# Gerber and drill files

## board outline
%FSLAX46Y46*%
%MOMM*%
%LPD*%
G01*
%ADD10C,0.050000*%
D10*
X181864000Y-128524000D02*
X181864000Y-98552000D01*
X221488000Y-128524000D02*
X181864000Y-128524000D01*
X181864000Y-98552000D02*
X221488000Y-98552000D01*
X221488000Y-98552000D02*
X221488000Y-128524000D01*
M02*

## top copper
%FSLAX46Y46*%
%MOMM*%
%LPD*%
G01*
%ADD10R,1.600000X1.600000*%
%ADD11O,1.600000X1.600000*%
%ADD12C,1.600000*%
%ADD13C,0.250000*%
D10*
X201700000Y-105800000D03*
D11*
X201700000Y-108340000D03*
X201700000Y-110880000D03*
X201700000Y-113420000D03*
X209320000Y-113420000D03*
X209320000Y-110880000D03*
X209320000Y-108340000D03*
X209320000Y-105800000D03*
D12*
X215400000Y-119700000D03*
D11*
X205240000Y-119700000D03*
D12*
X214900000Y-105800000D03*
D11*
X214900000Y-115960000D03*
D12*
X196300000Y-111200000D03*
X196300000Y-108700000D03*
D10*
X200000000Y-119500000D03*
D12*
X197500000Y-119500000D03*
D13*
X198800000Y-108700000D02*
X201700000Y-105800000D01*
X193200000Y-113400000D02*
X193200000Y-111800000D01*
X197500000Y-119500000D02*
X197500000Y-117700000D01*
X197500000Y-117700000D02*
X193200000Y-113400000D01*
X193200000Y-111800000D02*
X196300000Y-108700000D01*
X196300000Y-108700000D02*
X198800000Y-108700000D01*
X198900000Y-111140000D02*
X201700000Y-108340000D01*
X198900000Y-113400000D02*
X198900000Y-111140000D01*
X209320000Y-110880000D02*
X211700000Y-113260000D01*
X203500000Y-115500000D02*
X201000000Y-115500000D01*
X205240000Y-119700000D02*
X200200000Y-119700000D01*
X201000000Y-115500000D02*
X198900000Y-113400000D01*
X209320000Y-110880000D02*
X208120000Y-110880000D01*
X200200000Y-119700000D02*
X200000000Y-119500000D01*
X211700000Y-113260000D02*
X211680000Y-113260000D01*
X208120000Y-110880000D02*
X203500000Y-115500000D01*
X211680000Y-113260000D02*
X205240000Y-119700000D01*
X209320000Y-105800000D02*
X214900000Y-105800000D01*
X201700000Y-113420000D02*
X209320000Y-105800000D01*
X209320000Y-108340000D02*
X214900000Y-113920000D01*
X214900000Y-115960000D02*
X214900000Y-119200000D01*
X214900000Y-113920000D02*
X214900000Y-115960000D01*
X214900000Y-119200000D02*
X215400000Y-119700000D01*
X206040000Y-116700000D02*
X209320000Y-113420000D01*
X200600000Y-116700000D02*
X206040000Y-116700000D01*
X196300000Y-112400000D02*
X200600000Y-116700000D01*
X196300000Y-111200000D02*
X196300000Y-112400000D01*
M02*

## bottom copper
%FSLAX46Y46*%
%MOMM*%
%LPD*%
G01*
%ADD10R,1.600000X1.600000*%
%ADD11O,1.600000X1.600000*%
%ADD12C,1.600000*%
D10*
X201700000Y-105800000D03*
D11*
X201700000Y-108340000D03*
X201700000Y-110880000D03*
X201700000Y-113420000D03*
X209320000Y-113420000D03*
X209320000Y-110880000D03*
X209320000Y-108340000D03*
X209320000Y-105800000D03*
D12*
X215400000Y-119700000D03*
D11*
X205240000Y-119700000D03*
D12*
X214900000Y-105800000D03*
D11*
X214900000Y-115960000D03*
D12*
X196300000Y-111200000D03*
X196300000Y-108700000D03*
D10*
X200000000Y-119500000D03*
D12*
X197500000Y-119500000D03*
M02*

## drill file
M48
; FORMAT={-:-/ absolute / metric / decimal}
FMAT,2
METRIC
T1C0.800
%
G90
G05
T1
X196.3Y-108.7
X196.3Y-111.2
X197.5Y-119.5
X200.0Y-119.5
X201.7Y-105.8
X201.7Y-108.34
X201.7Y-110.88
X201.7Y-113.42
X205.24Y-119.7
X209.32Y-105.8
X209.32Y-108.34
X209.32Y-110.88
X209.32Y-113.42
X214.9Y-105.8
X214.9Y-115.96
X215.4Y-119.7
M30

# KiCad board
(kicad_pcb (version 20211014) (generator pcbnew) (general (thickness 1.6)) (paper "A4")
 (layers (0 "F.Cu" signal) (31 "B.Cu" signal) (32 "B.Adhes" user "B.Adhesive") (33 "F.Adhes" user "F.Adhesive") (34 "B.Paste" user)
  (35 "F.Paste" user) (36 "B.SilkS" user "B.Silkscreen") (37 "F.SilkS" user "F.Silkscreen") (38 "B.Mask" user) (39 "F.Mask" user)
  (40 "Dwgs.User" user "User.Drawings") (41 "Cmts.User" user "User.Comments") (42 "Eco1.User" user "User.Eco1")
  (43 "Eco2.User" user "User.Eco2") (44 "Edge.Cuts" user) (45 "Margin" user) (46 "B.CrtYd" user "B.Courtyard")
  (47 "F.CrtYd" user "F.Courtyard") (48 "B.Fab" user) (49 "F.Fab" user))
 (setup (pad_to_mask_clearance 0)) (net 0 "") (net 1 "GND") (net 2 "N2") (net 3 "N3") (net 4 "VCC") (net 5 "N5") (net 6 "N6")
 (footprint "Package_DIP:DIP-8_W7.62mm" (layer "F.Cu") (at 201.7 105.8)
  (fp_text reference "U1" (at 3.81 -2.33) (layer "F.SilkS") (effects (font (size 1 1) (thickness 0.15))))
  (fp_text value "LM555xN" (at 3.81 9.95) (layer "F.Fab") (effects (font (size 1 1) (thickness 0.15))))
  (pad "1" thru_hole rect locked (at 0 0) (size 1.6 1.6) (drill 0.8) (layers *.Cu *.Mask) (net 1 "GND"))
  (pad "2" thru_hole oval locked (at 0 2.54) (size 1.6 1.6) (drill 0.8) (layers *.Cu *.Mask) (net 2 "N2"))
  (pad "3" thru_hole oval locked (at 0 5.08) (size 1.6 1.6) (drill 0.8) (layers *.Cu *.Mask) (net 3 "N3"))
  (pad "4" thru_hole oval locked (at 0 7.62) (size 1.6 1.6) (drill 0.8) (layers *.Cu *.Mask) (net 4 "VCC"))
  (pad "5" thru_hole oval locked (at 7.62 7.62) (size 1.6 1.6) (drill 0.8) (layers *.Cu *.Mask) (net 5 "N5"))
  (pad "6" thru_hole oval locked (at 7.62 5.08) (size 1.6 1.6) (drill 0.8) (layers *.Cu *.Mask) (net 2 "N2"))
  (pad "7" thru_hole oval locked (at 7.62 2.54) (size 1.6 1.6) (drill 0.8) (layers *.Cu *.Mask) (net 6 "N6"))
  (pad "8" thru_hole oval locked (at 7.62 0) (size 1.6 1.6) (drill 0.8) (layers *.Cu *.Mask) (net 4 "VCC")))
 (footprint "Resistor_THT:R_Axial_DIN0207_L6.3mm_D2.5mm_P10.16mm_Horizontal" (layer "F.Cu") (at 215.4 119.7 180)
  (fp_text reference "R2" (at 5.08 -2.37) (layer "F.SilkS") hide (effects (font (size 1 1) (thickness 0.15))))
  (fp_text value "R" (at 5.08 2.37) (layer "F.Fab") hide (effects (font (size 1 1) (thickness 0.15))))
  (pad "1" thru_hole circle locked (at 0 0 180) (size 1.6 1.6) (drill 0.8) (layers *.Cu *.Mask) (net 6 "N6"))
  (pad "2" thru_hole oval locked (at 10.16 0 180) (size 1.6 1.6) (drill 0.8) (layers *.Cu *.Mask) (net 2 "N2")))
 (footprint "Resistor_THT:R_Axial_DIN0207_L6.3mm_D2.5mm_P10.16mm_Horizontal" (layer "F.Cu") (at 214.9 105.8 -90)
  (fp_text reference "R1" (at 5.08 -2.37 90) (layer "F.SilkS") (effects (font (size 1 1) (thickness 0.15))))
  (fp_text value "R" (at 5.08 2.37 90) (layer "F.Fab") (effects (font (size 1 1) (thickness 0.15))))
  (pad "1" thru_hole circle locked (at 0 0 270) (size 1.6 1.6) (drill 0.8) (layers *.Cu *.Mask) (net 4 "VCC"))
  (pad "2" thru_hole oval locked (at 10.16 0 270) (size 1.6 1.6) (drill 0.8) (layers *.Cu *.Mask) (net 6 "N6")))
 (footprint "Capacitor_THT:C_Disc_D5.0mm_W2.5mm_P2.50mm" (layer "F.Cu") (at 196.3 111.2 90)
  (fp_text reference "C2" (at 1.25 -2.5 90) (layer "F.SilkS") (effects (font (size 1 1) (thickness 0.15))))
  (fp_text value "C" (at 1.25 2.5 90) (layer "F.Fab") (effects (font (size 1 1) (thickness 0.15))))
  (pad "1" thru_hole circle locked (at 0 0 90) (size 1.6 1.6) (drill 0.8) (layers *.Cu *.Mask) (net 5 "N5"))
  (pad "2" thru_hole circle locked (at 2.5 0 90) (size 1.6 1.6) (drill 0.8) (layers *.Cu *.Mask) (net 1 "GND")))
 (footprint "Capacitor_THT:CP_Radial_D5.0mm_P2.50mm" (layer "F.Cu") (at 200 119.5 180)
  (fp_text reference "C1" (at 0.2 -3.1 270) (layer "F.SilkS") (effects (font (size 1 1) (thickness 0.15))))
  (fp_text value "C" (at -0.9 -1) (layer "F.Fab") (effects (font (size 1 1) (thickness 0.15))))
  (pad "1" thru_hole rect locked (at 0 0 180) (size 1.6 1.6) (drill 0.8) (layers *.Cu *.Mask) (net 2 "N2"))
  (pad "2" thru_hole circle locked (at 2.5 0 180) (size 1.6 1.6) (drill 0.8) (layers *.Cu *.Mask) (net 1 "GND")))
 (gr_line (start 181.864 128.524) (end 181.864 98.552) (layer "Edge.Cuts") (width 0.05))
 (gr_line (start 221.488 128.524) (end 181.864 128.524) (layer "Edge.Cuts") (width 0.05))
 (gr_line (start 181.864 98.552) (end 221.488 98.552) (layer "Edge.Cuts") (width 0.05))
 (gr_line (start 221.488 98.552) (end 221.488 128.524) (layer "Edge.Cuts") (width 0.05))
 (segment (start 198.8 108.7) (end 201.7 105.8) (width 0.25) (layer "F.Cu") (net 1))
 (segment (start 193.2 113.4) (end 193.2 111.8) (width 0.25) (layer "F.Cu") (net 1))
 (segment (start 197.5 119.5) (end 197.5 117.7) (width 0.25) (layer "F.Cu") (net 1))
 (segment (start 197.5 117.7) (end 193.2 113.4) (width 0.25) (layer "F.Cu") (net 1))
 (segment (start 193.2 111.8) (end 196.3 108.7) (width 0.25) (layer "F.Cu") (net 1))
 (segment (start 196.3 108.7) (end 198.8 108.7) (width 0.25) (layer "F.Cu") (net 1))
 (segment (start 198.9 111.14) (end 201.7 108.34) (width 0.25) (layer "F.Cu") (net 2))
 (segment (start 198.9 113.4) (end 198.9 111.14) (width 0.25) (layer "F.Cu") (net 2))
 (segment (start 209.32 110.88) (end 211.7 113.26) (width 0.25) (layer "F.Cu") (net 2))
 (segment (start 203.5 115.5) (end 201 115.5) (width 0.25) (layer "F.Cu") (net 2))
 (segment (start 205.24 119.7) (end 200.2 119.7) (width 0.25) (layer "F.Cu") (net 2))
 (segment (start 201 115.5) (end 198.9 113.4) (width 0.25) (layer "F.Cu") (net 2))
 (segment (start 209.32 110.88) (end 208.12 110.88) (width 0.25) (layer "F.Cu") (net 2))
 (segment (start 200.2 119.7) (end 200 119.5) (width 0.25) (layer "F.Cu") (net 2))
 (segment (start 211.7 113.26) (end 211.68 113.26) (width 0.25) (layer "F.Cu") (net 2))
 (segment (start 208.12 110.88) (end 203.5 115.5) (width 0.25) (layer "F.Cu") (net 2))
 (segment (start 211.68 113.26) (end 205.24 119.7) (width 0.25) (layer "F.Cu") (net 2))
 (segment (start 209.32 105.8) (end 214.9 105.8) (width 0.25) (layer "F.Cu") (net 4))
 (segment (start 201.7 113.42) (end 209.32 105.8) (width 0.25) (layer "F.Cu") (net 4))
 (segment (start 209.32 108.34) (end 214.9 113.92) (width 0.25) (layer "F.Cu") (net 6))
 (segment (start 214.9 115.96) (end 214.9 119.2) (width 0.25) (layer "F.Cu") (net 6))
 (segment (start 214.9 113.92) (end 214.9 115.96) (width 0.25) (layer "F.Cu") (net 6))
 (segment (start 214.9 119.2) (end 215.4 119.7) (width 0.25) (layer "F.Cu") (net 6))
 (segment (start 206.04 116.7) (end 209.32 113.42) (width 0.25) (layer "F.Cu") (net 5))
 (segment (start 200.6 116.7) (end 206.04 116.7) (width 0.25) (layer "F.Cu") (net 5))
 (segment (start 196.3 112.4) (end 200.6 116.7) (width 0.25) (layer "F.Cu") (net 5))
 (segment (start 196.3 111.2) (end 196.3 112.4) (width 0.25) (layer "F.Cu") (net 5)))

